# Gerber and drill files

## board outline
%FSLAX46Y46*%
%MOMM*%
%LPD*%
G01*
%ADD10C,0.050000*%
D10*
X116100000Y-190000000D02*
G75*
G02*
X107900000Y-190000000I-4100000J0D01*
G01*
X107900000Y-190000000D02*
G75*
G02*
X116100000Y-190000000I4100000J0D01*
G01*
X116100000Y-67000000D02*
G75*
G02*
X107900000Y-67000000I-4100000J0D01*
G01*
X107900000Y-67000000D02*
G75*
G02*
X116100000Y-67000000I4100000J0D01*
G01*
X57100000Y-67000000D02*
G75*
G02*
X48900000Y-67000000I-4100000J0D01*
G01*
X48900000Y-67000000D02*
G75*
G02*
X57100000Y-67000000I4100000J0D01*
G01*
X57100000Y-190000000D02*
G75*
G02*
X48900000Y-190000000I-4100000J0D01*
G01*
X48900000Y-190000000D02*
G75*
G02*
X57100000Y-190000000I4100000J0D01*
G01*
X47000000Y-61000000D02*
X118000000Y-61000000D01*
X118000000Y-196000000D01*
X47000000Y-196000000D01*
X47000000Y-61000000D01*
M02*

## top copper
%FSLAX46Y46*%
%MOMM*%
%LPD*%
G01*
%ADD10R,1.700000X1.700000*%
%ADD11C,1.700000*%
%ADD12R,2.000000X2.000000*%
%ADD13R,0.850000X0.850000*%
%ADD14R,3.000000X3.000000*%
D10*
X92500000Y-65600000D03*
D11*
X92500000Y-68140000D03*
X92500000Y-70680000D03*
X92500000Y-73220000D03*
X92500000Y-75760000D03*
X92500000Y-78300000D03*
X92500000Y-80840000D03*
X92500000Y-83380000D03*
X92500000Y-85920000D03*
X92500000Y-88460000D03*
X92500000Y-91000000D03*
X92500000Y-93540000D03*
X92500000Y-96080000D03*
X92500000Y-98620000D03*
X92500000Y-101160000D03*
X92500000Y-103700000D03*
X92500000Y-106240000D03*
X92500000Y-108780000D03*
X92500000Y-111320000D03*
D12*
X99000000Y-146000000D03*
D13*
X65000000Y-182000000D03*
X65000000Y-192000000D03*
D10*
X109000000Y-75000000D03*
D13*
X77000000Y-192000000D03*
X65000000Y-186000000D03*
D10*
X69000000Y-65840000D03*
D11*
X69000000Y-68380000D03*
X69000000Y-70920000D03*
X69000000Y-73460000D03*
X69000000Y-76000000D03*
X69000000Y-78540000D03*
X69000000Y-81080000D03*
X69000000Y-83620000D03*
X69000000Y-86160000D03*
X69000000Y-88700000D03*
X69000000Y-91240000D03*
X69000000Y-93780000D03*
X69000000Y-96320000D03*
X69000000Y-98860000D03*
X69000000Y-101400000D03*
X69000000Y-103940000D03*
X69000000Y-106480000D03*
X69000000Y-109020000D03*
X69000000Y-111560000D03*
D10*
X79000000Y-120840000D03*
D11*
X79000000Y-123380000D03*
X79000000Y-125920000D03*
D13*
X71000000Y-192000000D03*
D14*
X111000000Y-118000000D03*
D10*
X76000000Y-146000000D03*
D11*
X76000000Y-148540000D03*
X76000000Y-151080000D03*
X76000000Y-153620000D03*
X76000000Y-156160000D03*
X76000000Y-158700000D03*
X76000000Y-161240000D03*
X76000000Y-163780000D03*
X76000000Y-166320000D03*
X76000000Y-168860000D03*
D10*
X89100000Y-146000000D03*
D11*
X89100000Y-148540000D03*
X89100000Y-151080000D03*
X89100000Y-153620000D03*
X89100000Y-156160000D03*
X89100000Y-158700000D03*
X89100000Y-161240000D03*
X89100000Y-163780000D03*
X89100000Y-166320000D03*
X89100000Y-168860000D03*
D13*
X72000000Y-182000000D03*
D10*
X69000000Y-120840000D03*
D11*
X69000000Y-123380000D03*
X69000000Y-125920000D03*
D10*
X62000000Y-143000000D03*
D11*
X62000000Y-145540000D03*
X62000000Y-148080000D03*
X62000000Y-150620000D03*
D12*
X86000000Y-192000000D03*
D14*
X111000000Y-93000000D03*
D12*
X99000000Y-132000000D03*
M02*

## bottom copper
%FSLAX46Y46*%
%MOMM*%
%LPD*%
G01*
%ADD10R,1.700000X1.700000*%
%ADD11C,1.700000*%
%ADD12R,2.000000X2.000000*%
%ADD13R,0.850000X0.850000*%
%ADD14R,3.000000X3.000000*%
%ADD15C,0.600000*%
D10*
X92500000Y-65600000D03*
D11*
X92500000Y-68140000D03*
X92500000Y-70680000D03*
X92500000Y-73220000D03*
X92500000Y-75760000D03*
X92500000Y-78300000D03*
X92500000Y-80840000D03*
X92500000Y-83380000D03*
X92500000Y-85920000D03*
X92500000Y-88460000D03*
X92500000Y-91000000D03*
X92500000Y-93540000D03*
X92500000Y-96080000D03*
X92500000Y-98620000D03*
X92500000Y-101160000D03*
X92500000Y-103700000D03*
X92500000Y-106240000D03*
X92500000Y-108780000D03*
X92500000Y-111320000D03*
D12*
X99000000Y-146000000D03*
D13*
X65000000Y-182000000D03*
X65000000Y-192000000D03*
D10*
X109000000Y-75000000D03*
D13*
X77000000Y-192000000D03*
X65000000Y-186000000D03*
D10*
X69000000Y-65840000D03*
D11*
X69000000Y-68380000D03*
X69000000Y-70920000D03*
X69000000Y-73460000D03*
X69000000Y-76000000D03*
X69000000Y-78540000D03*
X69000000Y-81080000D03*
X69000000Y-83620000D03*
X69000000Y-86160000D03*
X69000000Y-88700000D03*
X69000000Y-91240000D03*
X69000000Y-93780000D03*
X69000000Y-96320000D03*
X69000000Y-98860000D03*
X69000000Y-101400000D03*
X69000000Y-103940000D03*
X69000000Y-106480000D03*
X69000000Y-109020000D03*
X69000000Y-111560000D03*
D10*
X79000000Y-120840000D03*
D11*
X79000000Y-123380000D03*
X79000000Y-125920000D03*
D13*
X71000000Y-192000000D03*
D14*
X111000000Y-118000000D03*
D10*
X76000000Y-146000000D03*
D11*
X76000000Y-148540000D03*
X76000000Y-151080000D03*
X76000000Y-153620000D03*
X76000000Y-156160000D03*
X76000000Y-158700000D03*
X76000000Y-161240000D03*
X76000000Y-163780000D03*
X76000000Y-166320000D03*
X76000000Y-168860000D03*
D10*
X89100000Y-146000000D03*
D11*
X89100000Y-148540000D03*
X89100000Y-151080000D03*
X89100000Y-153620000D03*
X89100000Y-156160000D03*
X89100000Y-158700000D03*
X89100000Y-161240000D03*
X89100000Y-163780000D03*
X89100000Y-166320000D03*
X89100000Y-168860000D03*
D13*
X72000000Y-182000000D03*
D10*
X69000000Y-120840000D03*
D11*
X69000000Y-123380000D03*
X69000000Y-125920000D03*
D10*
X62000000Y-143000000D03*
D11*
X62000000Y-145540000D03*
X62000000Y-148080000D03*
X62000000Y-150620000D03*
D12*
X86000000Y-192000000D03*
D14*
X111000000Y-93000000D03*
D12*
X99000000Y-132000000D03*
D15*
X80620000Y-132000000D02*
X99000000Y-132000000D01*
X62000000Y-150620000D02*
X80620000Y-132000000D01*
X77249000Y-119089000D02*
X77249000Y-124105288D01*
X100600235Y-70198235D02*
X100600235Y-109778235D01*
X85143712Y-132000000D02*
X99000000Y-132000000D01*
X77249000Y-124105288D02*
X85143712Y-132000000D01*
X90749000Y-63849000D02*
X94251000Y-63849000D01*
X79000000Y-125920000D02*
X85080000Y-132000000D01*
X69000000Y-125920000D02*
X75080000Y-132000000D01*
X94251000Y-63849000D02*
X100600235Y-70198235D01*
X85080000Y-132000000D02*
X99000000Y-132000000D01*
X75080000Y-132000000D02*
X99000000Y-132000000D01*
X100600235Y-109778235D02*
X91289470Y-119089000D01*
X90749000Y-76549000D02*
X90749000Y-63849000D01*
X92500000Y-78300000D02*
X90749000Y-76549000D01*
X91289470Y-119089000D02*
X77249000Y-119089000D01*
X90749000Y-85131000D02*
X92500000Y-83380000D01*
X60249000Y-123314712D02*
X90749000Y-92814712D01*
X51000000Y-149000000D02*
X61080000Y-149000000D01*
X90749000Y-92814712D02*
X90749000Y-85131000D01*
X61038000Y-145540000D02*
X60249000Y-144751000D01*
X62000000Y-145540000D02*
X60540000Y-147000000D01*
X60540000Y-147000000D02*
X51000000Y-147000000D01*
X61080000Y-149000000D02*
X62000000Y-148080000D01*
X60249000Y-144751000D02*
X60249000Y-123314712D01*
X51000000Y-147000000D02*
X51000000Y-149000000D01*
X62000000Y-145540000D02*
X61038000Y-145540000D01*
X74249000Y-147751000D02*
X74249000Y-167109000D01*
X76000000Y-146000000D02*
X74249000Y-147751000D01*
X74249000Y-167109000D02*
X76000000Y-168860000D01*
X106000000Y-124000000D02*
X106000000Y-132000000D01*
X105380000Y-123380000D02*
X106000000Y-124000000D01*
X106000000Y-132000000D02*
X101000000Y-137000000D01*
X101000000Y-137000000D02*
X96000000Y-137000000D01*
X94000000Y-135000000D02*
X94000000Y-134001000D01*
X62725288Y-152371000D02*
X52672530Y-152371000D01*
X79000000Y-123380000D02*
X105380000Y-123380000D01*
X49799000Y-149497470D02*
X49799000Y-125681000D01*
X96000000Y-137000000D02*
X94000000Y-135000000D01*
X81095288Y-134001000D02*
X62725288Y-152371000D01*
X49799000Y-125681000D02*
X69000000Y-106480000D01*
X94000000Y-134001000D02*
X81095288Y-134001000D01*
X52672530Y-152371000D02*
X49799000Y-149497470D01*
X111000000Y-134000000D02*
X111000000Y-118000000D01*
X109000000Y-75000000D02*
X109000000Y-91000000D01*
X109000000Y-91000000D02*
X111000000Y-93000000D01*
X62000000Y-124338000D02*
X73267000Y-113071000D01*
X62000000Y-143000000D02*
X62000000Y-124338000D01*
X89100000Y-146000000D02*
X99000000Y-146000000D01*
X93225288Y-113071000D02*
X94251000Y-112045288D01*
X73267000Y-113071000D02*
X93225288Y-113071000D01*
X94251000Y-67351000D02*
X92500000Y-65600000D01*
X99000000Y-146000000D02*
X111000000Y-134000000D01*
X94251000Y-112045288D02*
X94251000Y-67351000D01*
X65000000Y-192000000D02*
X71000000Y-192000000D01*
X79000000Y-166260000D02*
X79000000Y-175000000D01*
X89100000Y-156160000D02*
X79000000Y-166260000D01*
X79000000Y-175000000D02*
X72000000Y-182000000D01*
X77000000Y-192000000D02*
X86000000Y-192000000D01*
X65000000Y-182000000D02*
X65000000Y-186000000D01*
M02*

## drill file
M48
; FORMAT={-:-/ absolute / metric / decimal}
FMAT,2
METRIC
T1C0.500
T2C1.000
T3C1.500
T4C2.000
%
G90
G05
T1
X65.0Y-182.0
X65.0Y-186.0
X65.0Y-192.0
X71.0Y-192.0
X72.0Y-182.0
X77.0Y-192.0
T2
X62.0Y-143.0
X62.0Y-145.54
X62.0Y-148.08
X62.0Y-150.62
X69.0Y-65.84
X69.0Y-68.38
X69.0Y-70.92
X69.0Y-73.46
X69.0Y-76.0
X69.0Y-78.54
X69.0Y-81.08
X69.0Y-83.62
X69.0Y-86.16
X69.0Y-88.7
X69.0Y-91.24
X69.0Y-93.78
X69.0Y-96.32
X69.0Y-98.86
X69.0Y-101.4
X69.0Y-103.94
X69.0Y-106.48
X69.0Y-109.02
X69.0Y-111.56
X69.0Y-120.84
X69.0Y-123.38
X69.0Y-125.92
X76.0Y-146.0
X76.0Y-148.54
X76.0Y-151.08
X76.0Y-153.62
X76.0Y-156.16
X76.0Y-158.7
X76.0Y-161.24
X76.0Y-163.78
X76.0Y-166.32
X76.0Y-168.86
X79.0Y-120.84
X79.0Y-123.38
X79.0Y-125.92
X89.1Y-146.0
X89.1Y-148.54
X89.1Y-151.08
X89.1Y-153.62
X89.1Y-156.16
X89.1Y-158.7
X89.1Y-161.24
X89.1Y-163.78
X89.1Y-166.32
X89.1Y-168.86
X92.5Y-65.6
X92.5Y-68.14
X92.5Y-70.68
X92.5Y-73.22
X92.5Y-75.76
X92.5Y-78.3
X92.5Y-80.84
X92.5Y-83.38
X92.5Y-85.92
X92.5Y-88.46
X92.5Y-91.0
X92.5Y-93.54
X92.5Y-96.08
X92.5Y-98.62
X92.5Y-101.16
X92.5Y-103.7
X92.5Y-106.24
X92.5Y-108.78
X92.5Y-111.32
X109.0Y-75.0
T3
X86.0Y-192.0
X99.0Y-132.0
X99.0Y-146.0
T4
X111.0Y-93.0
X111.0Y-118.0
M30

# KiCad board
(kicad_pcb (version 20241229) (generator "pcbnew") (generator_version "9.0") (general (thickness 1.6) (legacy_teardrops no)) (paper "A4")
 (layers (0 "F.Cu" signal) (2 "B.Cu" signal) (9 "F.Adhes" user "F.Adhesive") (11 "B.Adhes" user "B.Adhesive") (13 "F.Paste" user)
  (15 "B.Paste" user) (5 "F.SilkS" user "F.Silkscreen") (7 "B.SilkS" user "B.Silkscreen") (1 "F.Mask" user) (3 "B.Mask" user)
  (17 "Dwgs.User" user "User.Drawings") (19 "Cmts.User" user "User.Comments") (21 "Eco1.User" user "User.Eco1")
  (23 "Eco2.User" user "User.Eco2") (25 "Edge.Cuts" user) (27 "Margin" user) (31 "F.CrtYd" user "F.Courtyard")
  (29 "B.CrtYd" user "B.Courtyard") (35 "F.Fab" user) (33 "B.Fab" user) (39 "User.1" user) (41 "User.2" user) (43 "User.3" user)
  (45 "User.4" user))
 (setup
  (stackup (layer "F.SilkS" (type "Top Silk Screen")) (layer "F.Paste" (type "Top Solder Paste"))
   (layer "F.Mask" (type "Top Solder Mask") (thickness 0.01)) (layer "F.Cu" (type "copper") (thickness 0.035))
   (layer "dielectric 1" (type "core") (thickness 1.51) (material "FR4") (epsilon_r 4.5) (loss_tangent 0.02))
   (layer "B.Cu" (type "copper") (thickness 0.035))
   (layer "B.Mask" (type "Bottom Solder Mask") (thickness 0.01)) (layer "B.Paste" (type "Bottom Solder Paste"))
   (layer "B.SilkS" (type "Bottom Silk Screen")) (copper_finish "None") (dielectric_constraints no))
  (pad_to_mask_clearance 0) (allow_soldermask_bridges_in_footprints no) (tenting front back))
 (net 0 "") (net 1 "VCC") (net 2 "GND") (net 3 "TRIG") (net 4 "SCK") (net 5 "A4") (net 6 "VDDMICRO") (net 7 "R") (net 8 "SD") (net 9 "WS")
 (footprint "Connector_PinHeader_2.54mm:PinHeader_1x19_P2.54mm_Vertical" (layer "F.Cu") (at 92.5 65.6)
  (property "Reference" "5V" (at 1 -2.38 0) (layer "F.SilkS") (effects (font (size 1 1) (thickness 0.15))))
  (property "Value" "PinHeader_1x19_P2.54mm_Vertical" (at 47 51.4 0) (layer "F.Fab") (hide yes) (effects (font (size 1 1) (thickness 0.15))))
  (pad "1" thru_hole rect (at 0 0) (size 1.7 1.7) (drill 1) (layers "*.Cu" "*.Mask") (remove_unused_layers no) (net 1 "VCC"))
  (pad "2" thru_hole circle (at 0 2.54) (size 1.7 1.7) (drill 1) (layers "*.Cu" "*.Mask") (remove_unused_layers no))
  (pad "3" thru_hole circle (at 0 5.08) (size 1.7 1.7) (drill 1) (layers "*.Cu" "*.Mask") (remove_unused_layers no))
  (pad "4" thru_hole circle (at 0 7.62) (size 1.7 1.7) (drill 1) (layers "*.Cu" "*.Mask") (remove_unused_layers no))
  (pad "5" thru_hole circle (at 0 10.16) (size 1.7 1.7) (drill 1) (layers "*.Cu" "*.Mask") (remove_unused_layers no))
  (pad "6" thru_hole circle (at 0 12.7) (size 1.7 1.7) (drill 1) (layers "*.Cu" "*.Mask") (remove_unused_layers no) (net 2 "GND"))
  (pad "7" thru_hole circle (at 0 15.24) (size 1.7 1.7) (drill 1) (layers "*.Cu" "*.Mask") (remove_unused_layers no))
  (pad "8" thru_hole circle (at 0 17.78) (size 1.7 1.7) (drill 1) (layers "*.Cu" "*.Mask") (remove_unused_layers no) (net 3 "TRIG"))
  (pad "9" thru_hole circle (at 0 20.32) (size 1.7 1.7) (drill 1) (layers "*.Cu" "*.Mask") (remove_unused_layers no))
  (pad "10" thru_hole circle (at 0 22.86) (size 1.7 1.7) (drill 1) (layers "*.Cu" "*.Mask") (remove_unused_layers no) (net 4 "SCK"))
  (pad "11" thru_hole circle (at 0 25.4) (size 1.7 1.7) (drill 1) (layers "*.Cu" "*.Mask") (remove_unused_layers no))
  (pad "12" thru_hole circle (at 0 27.94) (size 1.7 1.7) (drill 1) (layers "*.Cu" "*.Mask") (remove_unused_layers no))
  (pad "13" thru_hole circle (at 0 30.48) (size 1.7 1.7) (drill 1) (layers "*.Cu" "*.Mask") (remove_unused_layers no) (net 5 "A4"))
  (pad "14" thru_hole circle (at 0 33.02) (size 1.7 1.7) (drill 1) (layers "*.Cu" "*.Mask") (remove_unused_layers no))
  (pad "15" thru_hole circle (at 0 35.56) (size 1.7 1.7) (drill 1) (layers "*.Cu" "*.Mask") (remove_unused_layers no))
  (pad "16" thru_hole circle (at 0 38.1) (size 1.7 1.7) (drill 1) (layers "*.Cu" "*.Mask") (remove_unused_layers no))
  (pad "17" thru_hole circle (at 0 40.64) (size 1.7 1.7) (drill 1) (layers "*.Cu" "*.Mask") (remove_unused_layers no))
  (pad "18" thru_hole circle (at 0 43.18) (size 1.7 1.7) (drill 1) (layers "*.Cu" "*.Mask") (remove_unused_layers no))
  (pad "19" thru_hole circle (at 0 45.72) (size 1.7 1.7) (drill 1) (layers "*.Cu" "*.Mask") (remove_unused_layers no) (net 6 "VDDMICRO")))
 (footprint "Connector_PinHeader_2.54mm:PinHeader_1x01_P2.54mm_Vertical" (layer "F.Cu") (at 99 146)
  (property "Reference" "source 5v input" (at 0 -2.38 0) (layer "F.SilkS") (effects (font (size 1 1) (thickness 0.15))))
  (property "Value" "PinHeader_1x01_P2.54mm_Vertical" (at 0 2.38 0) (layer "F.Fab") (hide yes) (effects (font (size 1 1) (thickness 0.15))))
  (pad "1" thru_hole rect (at 0 0) (size 2 2) (drill 1.5) (layers "*.Cu" "*.Mask") (remove_unused_layers no) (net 1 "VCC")))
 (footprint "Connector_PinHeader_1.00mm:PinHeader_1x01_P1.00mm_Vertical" (layer "F.Cu") (at 65 182)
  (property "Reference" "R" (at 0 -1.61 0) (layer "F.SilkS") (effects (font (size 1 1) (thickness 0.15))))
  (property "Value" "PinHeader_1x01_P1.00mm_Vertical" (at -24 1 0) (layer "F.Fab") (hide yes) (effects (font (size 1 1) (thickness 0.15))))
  (pad "1" thru_hole rect (at 0 0) (size 0.85 0.85) (drill 0.5) (layers "*.Cu" "*.Mask") (remove_unused_layers no) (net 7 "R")))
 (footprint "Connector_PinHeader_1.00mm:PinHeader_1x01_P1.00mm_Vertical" (layer "F.Cu") (at 65 192)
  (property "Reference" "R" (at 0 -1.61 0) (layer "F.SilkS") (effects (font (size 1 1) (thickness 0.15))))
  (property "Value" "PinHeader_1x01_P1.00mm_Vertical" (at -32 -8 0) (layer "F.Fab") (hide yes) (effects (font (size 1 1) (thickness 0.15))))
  (pad "1" thru_hole rect (at 0 0) (size 0.85 0.85) (drill 0.5) (layers "*.Cu" "*.Mask") (remove_unused_layers no) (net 7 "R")))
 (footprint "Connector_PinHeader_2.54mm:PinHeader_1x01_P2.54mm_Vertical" (layer "F.Cu") (at 109 75)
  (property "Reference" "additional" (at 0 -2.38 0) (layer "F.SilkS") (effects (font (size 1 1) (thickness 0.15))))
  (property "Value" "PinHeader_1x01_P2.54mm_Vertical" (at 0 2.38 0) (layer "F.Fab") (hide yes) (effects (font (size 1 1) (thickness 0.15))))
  (pad "1" thru_hole rect (at 0 0) (size 1.7 1.7) (drill 1) (layers "*.Cu" "*.Mask") (remove_unused_layers no) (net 1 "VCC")))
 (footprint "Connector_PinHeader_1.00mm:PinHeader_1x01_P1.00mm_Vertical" (layer "F.Cu") (at 77 192)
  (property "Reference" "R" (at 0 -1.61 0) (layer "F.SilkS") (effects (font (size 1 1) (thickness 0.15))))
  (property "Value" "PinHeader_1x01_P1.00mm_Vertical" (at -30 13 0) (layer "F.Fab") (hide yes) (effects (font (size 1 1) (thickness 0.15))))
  (pad "1" thru_hole rect (at 0 0) (size 0.85 0.85) (drill 0.5) (layers "*.Cu" "*.Mask") (remove_unused_layers no) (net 7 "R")))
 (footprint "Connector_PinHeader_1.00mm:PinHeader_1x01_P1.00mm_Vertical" (layer "F.Cu") (at 65 186)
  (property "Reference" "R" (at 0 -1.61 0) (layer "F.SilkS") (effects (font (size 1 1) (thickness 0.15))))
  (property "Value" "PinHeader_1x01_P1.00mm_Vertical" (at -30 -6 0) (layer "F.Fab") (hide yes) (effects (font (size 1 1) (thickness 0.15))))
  (pad "1" thru_hole rect (at 0 0) (size 0.85 0.85) (drill 0.5) (layers "*.Cu" "*.Mask") (remove_unused_layers no) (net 7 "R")))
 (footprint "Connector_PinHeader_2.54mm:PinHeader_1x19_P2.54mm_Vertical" (layer "F.Cu") (at 69 65.84)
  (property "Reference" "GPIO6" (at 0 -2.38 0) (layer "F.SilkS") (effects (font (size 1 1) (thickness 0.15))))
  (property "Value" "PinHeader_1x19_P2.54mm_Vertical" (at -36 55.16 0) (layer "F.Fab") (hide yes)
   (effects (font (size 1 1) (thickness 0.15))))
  (pad "1" thru_hole rect (at 0 0) (size 1.7 1.7) (drill 1) (layers "*.Cu" "*.Mask") (remove_unused_layers no))
  (pad "2" thru_hole circle (at 0 2.54) (size 1.7 1.7) (drill 1) (layers "*.Cu" "*.Mask") (remove_unused_layers no))
  (pad "3" thru_hole circle (at 0 5.08) (size 1.7 1.7) (drill 1) (layers "*.Cu" "*.Mask") (remove_unused_layers no))
  (pad "4" thru_hole circle (at 0 7.62) (size 1.7 1.7) (drill 1) (layers "*.Cu" "*.Mask") (remove_unused_layers no))
  (pad "5" thru_hole circle (at 0 10.16) (size 1.7 1.7) (drill 1) (layers "*.Cu" "*.Mask") (remove_unused_layers no))
  (pad "6" thru_hole circle (at 0 12.7) (size 1.7 1.7) (drill 1) (layers "*.Cu" "*.Mask") (remove_unused_layers no))
  (pad "7" thru_hole circle (at 0 15.24) (size 1.7 1.7) (drill 1) (layers "*.Cu" "*.Mask") (remove_unused_layers no))
  (pad "8" thru_hole circle (at 0 17.78) (size 1.7 1.7) (drill 1) (layers "*.Cu" "*.Mask") (remove_unused_layers no))
  (pad "9" thru_hole circle (at 0 20.32) (size 1.7 1.7) (drill 1) (layers "*.Cu" "*.Mask") (remove_unused_layers no))
  (pad "10" thru_hole circle (at 0 22.86) (size 1.7 1.7) (drill 1) (layers "*.Cu" "*.Mask") (remove_unused_layers no))
  (pad "11" thru_hole circle (at 0 25.4) (size 1.7 1.7) (drill 1) (layers "*.Cu" "*.Mask") (remove_unused_layers no))
  (pad "12" thru_hole circle (at 0 27.94) (size 1.7 1.7) (drill 1) (layers "*.Cu" "*.Mask") (remove_unused_layers no))
  (pad "13" thru_hole circle (at 0 30.48) (size 1.7 1.7) (drill 1) (layers "*.Cu" "*.Mask") (remove_unused_layers no))
  (pad "14" thru_hole circle (at 0 33.02) (size 1.7 1.7) (drill 1) (layers "*.Cu" "*.Mask") (remove_unused_layers no) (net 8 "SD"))
  (pad "15" thru_hole circle (at 0 35.56) (size 1.7 1.7) (drill 1) (layers "*.Cu" "*.Mask") (remove_unused_layers no))
  (pad "16" thru_hole circle (at 0 38.1) (size 1.7 1.7) (drill 1) (layers "*.Cu" "*.Mask") (remove_unused_layers no))
  (pad "17" thru_hole circle (at 0 40.64) (size 1.7 1.7) (drill 1) (layers "*.Cu" "*.Mask") (remove_unused_layers no) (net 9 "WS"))
  (pad "18" thru_hole circle (at 0 43.18) (size 1.7 1.7) (drill 1) (layers "*.Cu" "*.Mask") (remove_unused_layers no))
  (pad "19" thru_hole circle (at 0 45.72) (size 1.7 1.7) (drill 1) (layers "*.Cu" "*.Mask") (remove_unused_layers no)))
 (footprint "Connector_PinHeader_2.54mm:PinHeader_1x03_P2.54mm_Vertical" (layer "F.Cu") (at 79 120.84)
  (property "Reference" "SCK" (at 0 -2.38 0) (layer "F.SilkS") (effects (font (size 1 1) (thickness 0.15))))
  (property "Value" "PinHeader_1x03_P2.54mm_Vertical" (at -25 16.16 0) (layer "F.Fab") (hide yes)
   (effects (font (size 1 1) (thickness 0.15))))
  (pad "1" thru_hole rect (at 0 0) (size 1.7 1.7) (drill 1) (layers "*.Cu" "*.Mask") (remove_unused_layers no) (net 4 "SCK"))
  (pad "2" thru_hole circle (at 0 2.54) (size 1.7 1.7) (drill 1) (layers "*.Cu" "*.Mask") (remove_unused_layers no) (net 9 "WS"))
  (pad "3" thru_hole circle (at 0 5.08) (size 1.7 1.7) (drill 1) (layers "*.Cu" "*.Mask") (remove_unused_layers no) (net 2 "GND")))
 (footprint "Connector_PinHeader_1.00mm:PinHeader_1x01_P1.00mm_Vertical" (layer "F.Cu") (at 71 192)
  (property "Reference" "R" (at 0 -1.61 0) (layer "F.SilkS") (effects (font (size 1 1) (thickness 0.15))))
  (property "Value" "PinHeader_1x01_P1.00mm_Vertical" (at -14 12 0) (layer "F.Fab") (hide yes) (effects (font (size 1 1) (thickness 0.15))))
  (pad "1" thru_hole rect (at 0 0) (size 0.85 0.85) (drill 0.5) (layers "*.Cu" "*.Mask") (remove_unused_layers no) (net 7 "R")))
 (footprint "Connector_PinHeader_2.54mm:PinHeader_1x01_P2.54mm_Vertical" (layer "F.Cu") (at 111 118)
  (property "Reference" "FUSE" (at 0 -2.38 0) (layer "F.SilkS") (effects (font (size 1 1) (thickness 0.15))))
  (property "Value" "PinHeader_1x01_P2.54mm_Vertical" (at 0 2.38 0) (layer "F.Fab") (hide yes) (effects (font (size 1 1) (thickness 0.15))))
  (pad "1" thru_hole rect (at 0 0) (size 3 3) (drill 2) (layers "*.Cu" "*.Mask") (remove_unused_layers no) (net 1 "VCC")))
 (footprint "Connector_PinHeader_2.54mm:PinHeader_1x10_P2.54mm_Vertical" (layer "F.Cu") (at 76 146)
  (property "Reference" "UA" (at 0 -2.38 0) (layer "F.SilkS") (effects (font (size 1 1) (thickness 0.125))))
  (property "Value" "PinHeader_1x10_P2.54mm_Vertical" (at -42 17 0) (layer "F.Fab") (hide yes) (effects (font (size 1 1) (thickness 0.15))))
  (pad "1" thru_hole rect (at 0 0) (size 1.7 1.7) (drill 1) (layers "*.Cu" "*.Mask") (remove_unused_layers no) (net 6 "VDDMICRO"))
  (pad "2" thru_hole circle (at 0 2.54) (size 1.7 1.7) (drill 1) (layers "*.Cu" "*.Mask") (remove_unused_layers no))
  (pad "3" thru_hole circle (at 0 5.08) (size 1.7 1.7) (drill 1) (layers "*.Cu" "*.Mask") (remove_unused_layers no))
  (pad "4" thru_hole circle (at 0 7.62) (size 1.7 1.7) (drill 1) (layers "*.Cu" "*.Mask") (remove_unused_layers no))
  (pad "5" thru_hole circle (at 0 10.16) (size 1.7 1.7) (drill 1) (layers "*.Cu" "*.Mask") (remove_unused_layers no) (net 5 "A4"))
  (pad "6" thru_hole circle (at 0 12.7) (size 1.7 1.7) (drill 1) (layers "*.Cu" "*.Mask") (remove_unused_layers no))
  (pad "7" thru_hole circle (at 0 15.24) (size 1.7 1.7) (drill 1) (layers "*.Cu" "*.Mask") (remove_unused_layers no))
  (pad "8" thru_hole circle (at 0 17.78) (size 1.7 1.7) (drill 1) (layers "*.Cu" "*.Mask") (remove_unused_layers no))
  (pad "9" thru_hole circle (at 0 20.32) (size 1.7 1.7) (drill 1) (layers "*.Cu" "*.Mask") (remove_unused_layers no))
  (pad "10" thru_hole circle (at 0 22.86) (size 1.7 1.7) (drill 1) (layers "*.Cu" "*.Mask") (remove_unused_layers no) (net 6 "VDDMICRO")))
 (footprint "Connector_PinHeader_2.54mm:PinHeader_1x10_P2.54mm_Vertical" (layer "F.Cu") (at 89.1 146)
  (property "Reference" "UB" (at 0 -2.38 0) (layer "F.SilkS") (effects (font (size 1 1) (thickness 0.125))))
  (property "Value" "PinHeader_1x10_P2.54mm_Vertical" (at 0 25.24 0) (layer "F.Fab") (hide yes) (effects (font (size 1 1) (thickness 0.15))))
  (pad "1" thru_hole rect (at 0 0) (size 1.7 1.7) (drill 1) (layers "*.Cu" "*.Mask") (remove_unused_layers no) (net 1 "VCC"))
  (pad "2" thru_hole circle (at 0 2.54) (size 1.7 1.7) (drill 1) (layers "*.Cu" "*.Mask") (remove_unused_layers no))
  (pad "3" thru_hole circle (at 0 5.08) (size 1.7 1.7) (drill 1) (layers "*.Cu" "*.Mask") (remove_unused_layers no))
  (pad "4" thru_hole circle (at 0 7.62) (size 1.7 1.7) (drill 1) (layers "*.Cu" "*.Mask") (remove_unused_layers no))
  (pad "5" thru_hole circle (at 0 10.16) (size 1.7 1.7) (drill 1) (layers "*.Cu" "*.Mask") (remove_unused_layers no) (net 7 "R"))
  (pad "6" thru_hole circle (at 0 12.7) (size 1.7 1.7) (drill 1) (layers "*.Cu" "*.Mask") (remove_unused_layers no))
  (pad "7" thru_hole circle (at 0 15.24) (size 1.7 1.7) (drill 1) (layers "*.Cu" "*.Mask") (remove_unused_layers no))
  (pad "8" thru_hole circle (at 0 17.78) (size 1.7 1.7) (drill 1) (layers "*.Cu" "*.Mask") (remove_unused_layers no))
  (pad "9" thru_hole circle (at 0 20.32) (size 1.7 1.7) (drill 1) (layers "*.Cu" "*.Mask") (remove_unused_layers no))
  (pad "10" thru_hole circle (at 0 22.86) (size 1.7 1.7) (drill 1) (layers "*.Cu" "*.Mask") (remove_unused_layers no) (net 2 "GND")))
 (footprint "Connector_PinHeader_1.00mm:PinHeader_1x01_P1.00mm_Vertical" (layer "F.Cu") (at 72 182)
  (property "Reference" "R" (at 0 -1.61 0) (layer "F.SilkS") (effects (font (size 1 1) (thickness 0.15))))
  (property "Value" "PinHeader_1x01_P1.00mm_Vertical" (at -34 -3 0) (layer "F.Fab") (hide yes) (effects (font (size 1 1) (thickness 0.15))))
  (pad "1" thru_hole rect (at 0 0) (size 0.85 0.85) (drill 0.5) (layers "*.Cu" "*.Mask") (remove_unused_layers no) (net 7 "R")))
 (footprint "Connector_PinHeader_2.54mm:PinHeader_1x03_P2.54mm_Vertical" (layer "F.Cu") (at 69 120.84)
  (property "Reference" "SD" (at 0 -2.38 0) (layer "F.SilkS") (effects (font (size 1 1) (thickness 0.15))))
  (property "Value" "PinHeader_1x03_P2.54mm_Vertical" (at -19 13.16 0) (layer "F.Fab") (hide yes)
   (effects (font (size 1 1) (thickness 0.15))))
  (pad "1" thru_hole rect (at 0 0) (size 1.7 1.7) (drill 1) (layers "*.Cu" "*.Mask") (remove_unused_layers no) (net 8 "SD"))
  (pad "2" thru_hole circle (at 0 2.54) (size 1.7 1.7) (drill 1) (layers "*.Cu" "*.Mask") (remove_unused_layers no) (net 6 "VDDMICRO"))
  (pad "3" thru_hole circle (at 0 5.08) (size 1.7 1.7) (drill 1) (layers "*.Cu" "*.Mask") (remove_unused_layers no) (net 2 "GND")))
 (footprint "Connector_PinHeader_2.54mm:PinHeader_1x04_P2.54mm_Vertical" (layer "F.Cu") (at 62 143)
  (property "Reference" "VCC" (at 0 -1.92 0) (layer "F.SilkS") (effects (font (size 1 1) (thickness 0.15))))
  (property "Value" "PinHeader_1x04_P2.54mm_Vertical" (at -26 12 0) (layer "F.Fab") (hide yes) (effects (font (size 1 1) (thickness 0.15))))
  (pad "1" thru_hole rect (at 0 0) (size 1.7 1.7) (drill 1) (layers "*.Cu" "*.Mask") (remove_unused_layers no) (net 1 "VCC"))
  (pad "2" thru_hole circle (at 0 2.54) (size 1.7 1.7) (drill 1) (layers "*.Cu" "*.Mask") (remove_unused_layers no) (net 3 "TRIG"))
  (pad "3" thru_hole circle (at 0 5.08) (size 1.7 1.7) (drill 1) (layers "*.Cu" "*.Mask") (remove_unused_layers no) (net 3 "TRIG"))
  (pad "4" thru_hole circle (at 0 7.62) (size 1.7 1.7) (drill 1) (layers "*.Cu" "*.Mask") (remove_unused_layers no) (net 2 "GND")))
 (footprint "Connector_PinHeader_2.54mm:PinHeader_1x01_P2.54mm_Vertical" (layer "F.Cu") (at 86 192)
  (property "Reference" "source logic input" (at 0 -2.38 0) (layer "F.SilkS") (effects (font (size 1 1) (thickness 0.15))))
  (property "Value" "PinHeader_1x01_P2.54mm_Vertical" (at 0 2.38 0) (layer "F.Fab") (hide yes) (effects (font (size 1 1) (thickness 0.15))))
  (pad "1" thru_hole rect (at 0 0) (size 2 2) (drill 1.5) (layers "*.Cu" "*.Mask") (remove_unused_layers no) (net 7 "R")))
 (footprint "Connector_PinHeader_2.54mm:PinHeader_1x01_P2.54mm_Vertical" (layer "F.Cu") (at 111 93)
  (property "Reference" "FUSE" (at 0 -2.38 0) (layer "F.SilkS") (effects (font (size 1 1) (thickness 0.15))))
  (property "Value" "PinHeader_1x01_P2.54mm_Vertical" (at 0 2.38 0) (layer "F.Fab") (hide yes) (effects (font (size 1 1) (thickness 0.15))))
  (pad "1" thru_hole rect (at 0 0) (size 3 3) (drill 2) (layers "*.Cu" "*.Mask") (remove_unused_layers no) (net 1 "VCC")))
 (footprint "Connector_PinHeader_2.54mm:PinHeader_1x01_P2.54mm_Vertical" (layer "F.Cu") (at 99 132)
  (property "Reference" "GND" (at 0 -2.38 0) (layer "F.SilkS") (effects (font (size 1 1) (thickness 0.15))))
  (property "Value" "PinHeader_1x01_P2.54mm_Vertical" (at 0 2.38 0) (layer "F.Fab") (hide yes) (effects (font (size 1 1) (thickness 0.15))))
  (pad "1" thru_hole rect (at 0 0) (size 2 2) (drill 1.5) (layers "*.Cu" "*.Mask") (remove_unused_layers no) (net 2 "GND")))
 (gr_circle (center 112 190) (end 116.1 190) (stroke (width 0.05) (type solid)) (fill no) (layer "Edge.Cuts"))
 (gr_circle (center 112 67) (end 116.1 67) (stroke (width 0.05) (type solid)) (fill no) (layer "Edge.Cuts"))
 (gr_circle (center 53 67) (end 57.1 67) (stroke (width 0.05) (type solid)) (fill no) (layer "Edge.Cuts"))
 (gr_circle (center 53 190) (end 57.1 190) (stroke (width 0.05) (type solid)) (fill no) (layer "Edge.Cuts"))
 (gr_rect (start 47 61) (end 118 196) (stroke (width 0.05) (type default)) (fill no) (layer "Edge.Cuts"))
 (segment (start 80.62 132) (end 99 132) (width 0.6) (layer "B.Cu") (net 2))
 (segment (start 62 150.62) (end 80.62 132) (width 0.6) (layer "B.Cu") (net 2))
 (segment (start 77.249 119.089) (end 77.249 124.105288) (width 0.6) (layer "B.Cu") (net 2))
 (segment (start 100.600235 70.198235) (end 100.600235 109.778235) (width 0.6) (layer "B.Cu") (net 2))
 (segment (start 85.143712 132) (end 99 132) (width 0.6) (layer "B.Cu") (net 2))
 (segment (start 77.249 124.105288) (end 85.143712 132) (width 0.6) (layer "B.Cu") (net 2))
 (segment (start 90.749 63.849) (end 94.251 63.849) (width 0.6) (layer "B.Cu") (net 2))
 (segment (start 79 125.92) (end 85.08 132) (width 0.6) (layer "B.Cu") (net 2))
 (segment (start 69 125.92) (end 75.08 132) (width 0.6) (layer "B.Cu") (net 2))
 (segment (start 94.251 63.849) (end 100.600235 70.198235) (width 0.6) (layer "B.Cu") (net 2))
 (segment (start 85.08 132) (end 99 132) (width 0.6) (layer "B.Cu") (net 2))
 (segment (start 75.08 132) (end 99 132) (width 0.6) (layer "B.Cu") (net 2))
 (segment (start 100.600235 109.778235) (end 91.28947 119.089) (width 0.6) (layer "B.Cu") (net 2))
 (segment (start 90.749 76.549) (end 90.749 63.849) (width 0.6) (layer "B.Cu") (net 2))
 (segment (start 92.5 78.3) (end 90.749 76.549) (width 0.6) (layer "B.Cu") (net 2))
 (segment (start 91.28947 119.089) (end 77.249 119.089) (width 0.6) (layer "B.Cu") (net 2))
 (segment (start 90.749 85.131) (end 92.5 83.38) (width 0.6) (layer "B.Cu") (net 3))
 (segment (start 60.249 123.314712) (end 90.749 92.814712) (width 0.6) (layer "B.Cu") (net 3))
 (segment (start 51 149) (end 61.08 149) (width 0.6) (layer "B.Cu") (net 3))
 (segment (start 90.749 92.814712) (end 90.749 85.131) (width 0.6) (layer "B.Cu") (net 3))
 (segment (start 61.038 145.54) (end 60.249 144.751) (width 0.6) (layer "B.Cu") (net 3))
 (segment (start 62 145.54) (end 60.54 147) (width 0.6) (layer "B.Cu") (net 3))
 (segment (start 60.54 147) (end 51 147) (width 0.6) (layer "B.Cu") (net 3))
 (segment (start 61.08 149) (end 62 148.08) (width 0.6) (layer "B.Cu") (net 3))
 (segment (start 60.249 144.751) (end 60.249 123.314712) (width 0.6) (layer "B.Cu") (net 3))
 (segment (start 51 147) (end 51 149) (width 0.6) (layer "B.Cu") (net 3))
 (segment (start 62 145.54) (end 61.038 145.54) (width 0.6) (layer "B.Cu") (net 3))
 (segment (start 74.249 147.751) (end 74.249 167.109) (width 0.6) (layer "B.Cu") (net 6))
 (segment (start 76 146) (end 74.249 147.751) (width 0.6) (layer "B.Cu") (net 6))
 (segment (start 74.249 167.109) (end 76 168.86) (width 0.6) (layer "B.Cu") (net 6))
 (segment (start 106 124) (end 106 132) (width 0.6) (layer "B.Cu") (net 9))
 (segment (start 105.38 123.38) (end 106 124) (width 0.6) (layer "B.Cu") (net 9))
 (segment (start 106 132) (end 101 137) (width 0.6) (layer "B.Cu") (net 9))
 (segment (start 101 137) (end 96 137) (width 0.6) (layer "B.Cu") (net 9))
 (segment (start 94 135) (end 94 134.001) (width 0.6) (layer "B.Cu") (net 9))
 (segment (start 62.725288 152.371) (end 52.67253 152.371) (width 0.6) (layer "B.Cu") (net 9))
 (segment (start 79 123.38) (end 105.38 123.38) (width 0.6) (layer "B.Cu") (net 9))
 (segment (start 49.799 149.49747) (end 49.799 125.681) (width 0.6) (layer "B.Cu") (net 9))
 (segment (start 96 137) (end 94 135) (width 0.6) (layer "B.Cu") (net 9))
 (segment (start 81.095288 134.001) (end 62.725288 152.371) (width 0.6) (layer "B.Cu") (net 9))
 (segment (start 49.799 125.681) (end 69 106.48) (width 0.6) (layer "B.Cu") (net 9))
 (segment (start 94 134.001) (end 81.095288 134.001) (width 0.6) (layer "B.Cu") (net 9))
 (segment (start 52.67253 152.371) (end 49.799 149.49747) (width 0.6) (layer "B.Cu") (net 9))
 (segment (start 111 134) (end 111 118) (width 0.6) (layer "B.Cu") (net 1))
 (segment (start 109 75) (end 109 91) (width 0.6) (layer "B.Cu") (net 1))
 (segment (start 109 91) (end 111 93) (width 0.6) (layer "B.Cu") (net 1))
 (segment (start 62 124.338) (end 73.267 113.071) (width 0.6) (layer "B.Cu") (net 1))
 (segment (start 62 143) (end 62 124.338) (width 0.6) (layer "B.Cu") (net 1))
 (segment (start 89.1 146) (end 99 146) (width 0.6) (layer "B.Cu") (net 1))
 (segment (start 93.225288 113.071) (end 94.251 112.045288) (width 0.6) (layer "B.Cu") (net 1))
 (segment (start 73.267 113.071) (end 93.225288 113.071) (width 0.6) (layer "B.Cu") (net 1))
 (segment (start 94.251 67.351) (end 92.5 65.6) (width 0.6) (layer "B.Cu") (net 1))
 (segment (start 99 146) (end 111 134) (width 0.6) (layer "B.Cu") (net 1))
 (segment (start 94.251 112.045288) (end 94.251 67.351) (width 0.6) (layer "B.Cu") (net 1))
 (segment (start 65 192) (end 71 192) (width 0.6) (layer "B.Cu") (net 7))
 (segment (start 79 166.26) (end 79 175) (width 0.6) (layer "B.Cu") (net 7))
 (segment (start 89.1 156.16) (end 79 166.26) (width 0.6) (layer "B.Cu") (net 7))
 (segment (start 79 175) (end 72 182) (width 0.6) (layer "B.Cu") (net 7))
 (segment (start 77 192) (end 86 192) (width 0.6) (layer "B.Cu") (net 7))
 (segment (start 65 182) (end 65 186) (width 0.6) (layer "B.Cu") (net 7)))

